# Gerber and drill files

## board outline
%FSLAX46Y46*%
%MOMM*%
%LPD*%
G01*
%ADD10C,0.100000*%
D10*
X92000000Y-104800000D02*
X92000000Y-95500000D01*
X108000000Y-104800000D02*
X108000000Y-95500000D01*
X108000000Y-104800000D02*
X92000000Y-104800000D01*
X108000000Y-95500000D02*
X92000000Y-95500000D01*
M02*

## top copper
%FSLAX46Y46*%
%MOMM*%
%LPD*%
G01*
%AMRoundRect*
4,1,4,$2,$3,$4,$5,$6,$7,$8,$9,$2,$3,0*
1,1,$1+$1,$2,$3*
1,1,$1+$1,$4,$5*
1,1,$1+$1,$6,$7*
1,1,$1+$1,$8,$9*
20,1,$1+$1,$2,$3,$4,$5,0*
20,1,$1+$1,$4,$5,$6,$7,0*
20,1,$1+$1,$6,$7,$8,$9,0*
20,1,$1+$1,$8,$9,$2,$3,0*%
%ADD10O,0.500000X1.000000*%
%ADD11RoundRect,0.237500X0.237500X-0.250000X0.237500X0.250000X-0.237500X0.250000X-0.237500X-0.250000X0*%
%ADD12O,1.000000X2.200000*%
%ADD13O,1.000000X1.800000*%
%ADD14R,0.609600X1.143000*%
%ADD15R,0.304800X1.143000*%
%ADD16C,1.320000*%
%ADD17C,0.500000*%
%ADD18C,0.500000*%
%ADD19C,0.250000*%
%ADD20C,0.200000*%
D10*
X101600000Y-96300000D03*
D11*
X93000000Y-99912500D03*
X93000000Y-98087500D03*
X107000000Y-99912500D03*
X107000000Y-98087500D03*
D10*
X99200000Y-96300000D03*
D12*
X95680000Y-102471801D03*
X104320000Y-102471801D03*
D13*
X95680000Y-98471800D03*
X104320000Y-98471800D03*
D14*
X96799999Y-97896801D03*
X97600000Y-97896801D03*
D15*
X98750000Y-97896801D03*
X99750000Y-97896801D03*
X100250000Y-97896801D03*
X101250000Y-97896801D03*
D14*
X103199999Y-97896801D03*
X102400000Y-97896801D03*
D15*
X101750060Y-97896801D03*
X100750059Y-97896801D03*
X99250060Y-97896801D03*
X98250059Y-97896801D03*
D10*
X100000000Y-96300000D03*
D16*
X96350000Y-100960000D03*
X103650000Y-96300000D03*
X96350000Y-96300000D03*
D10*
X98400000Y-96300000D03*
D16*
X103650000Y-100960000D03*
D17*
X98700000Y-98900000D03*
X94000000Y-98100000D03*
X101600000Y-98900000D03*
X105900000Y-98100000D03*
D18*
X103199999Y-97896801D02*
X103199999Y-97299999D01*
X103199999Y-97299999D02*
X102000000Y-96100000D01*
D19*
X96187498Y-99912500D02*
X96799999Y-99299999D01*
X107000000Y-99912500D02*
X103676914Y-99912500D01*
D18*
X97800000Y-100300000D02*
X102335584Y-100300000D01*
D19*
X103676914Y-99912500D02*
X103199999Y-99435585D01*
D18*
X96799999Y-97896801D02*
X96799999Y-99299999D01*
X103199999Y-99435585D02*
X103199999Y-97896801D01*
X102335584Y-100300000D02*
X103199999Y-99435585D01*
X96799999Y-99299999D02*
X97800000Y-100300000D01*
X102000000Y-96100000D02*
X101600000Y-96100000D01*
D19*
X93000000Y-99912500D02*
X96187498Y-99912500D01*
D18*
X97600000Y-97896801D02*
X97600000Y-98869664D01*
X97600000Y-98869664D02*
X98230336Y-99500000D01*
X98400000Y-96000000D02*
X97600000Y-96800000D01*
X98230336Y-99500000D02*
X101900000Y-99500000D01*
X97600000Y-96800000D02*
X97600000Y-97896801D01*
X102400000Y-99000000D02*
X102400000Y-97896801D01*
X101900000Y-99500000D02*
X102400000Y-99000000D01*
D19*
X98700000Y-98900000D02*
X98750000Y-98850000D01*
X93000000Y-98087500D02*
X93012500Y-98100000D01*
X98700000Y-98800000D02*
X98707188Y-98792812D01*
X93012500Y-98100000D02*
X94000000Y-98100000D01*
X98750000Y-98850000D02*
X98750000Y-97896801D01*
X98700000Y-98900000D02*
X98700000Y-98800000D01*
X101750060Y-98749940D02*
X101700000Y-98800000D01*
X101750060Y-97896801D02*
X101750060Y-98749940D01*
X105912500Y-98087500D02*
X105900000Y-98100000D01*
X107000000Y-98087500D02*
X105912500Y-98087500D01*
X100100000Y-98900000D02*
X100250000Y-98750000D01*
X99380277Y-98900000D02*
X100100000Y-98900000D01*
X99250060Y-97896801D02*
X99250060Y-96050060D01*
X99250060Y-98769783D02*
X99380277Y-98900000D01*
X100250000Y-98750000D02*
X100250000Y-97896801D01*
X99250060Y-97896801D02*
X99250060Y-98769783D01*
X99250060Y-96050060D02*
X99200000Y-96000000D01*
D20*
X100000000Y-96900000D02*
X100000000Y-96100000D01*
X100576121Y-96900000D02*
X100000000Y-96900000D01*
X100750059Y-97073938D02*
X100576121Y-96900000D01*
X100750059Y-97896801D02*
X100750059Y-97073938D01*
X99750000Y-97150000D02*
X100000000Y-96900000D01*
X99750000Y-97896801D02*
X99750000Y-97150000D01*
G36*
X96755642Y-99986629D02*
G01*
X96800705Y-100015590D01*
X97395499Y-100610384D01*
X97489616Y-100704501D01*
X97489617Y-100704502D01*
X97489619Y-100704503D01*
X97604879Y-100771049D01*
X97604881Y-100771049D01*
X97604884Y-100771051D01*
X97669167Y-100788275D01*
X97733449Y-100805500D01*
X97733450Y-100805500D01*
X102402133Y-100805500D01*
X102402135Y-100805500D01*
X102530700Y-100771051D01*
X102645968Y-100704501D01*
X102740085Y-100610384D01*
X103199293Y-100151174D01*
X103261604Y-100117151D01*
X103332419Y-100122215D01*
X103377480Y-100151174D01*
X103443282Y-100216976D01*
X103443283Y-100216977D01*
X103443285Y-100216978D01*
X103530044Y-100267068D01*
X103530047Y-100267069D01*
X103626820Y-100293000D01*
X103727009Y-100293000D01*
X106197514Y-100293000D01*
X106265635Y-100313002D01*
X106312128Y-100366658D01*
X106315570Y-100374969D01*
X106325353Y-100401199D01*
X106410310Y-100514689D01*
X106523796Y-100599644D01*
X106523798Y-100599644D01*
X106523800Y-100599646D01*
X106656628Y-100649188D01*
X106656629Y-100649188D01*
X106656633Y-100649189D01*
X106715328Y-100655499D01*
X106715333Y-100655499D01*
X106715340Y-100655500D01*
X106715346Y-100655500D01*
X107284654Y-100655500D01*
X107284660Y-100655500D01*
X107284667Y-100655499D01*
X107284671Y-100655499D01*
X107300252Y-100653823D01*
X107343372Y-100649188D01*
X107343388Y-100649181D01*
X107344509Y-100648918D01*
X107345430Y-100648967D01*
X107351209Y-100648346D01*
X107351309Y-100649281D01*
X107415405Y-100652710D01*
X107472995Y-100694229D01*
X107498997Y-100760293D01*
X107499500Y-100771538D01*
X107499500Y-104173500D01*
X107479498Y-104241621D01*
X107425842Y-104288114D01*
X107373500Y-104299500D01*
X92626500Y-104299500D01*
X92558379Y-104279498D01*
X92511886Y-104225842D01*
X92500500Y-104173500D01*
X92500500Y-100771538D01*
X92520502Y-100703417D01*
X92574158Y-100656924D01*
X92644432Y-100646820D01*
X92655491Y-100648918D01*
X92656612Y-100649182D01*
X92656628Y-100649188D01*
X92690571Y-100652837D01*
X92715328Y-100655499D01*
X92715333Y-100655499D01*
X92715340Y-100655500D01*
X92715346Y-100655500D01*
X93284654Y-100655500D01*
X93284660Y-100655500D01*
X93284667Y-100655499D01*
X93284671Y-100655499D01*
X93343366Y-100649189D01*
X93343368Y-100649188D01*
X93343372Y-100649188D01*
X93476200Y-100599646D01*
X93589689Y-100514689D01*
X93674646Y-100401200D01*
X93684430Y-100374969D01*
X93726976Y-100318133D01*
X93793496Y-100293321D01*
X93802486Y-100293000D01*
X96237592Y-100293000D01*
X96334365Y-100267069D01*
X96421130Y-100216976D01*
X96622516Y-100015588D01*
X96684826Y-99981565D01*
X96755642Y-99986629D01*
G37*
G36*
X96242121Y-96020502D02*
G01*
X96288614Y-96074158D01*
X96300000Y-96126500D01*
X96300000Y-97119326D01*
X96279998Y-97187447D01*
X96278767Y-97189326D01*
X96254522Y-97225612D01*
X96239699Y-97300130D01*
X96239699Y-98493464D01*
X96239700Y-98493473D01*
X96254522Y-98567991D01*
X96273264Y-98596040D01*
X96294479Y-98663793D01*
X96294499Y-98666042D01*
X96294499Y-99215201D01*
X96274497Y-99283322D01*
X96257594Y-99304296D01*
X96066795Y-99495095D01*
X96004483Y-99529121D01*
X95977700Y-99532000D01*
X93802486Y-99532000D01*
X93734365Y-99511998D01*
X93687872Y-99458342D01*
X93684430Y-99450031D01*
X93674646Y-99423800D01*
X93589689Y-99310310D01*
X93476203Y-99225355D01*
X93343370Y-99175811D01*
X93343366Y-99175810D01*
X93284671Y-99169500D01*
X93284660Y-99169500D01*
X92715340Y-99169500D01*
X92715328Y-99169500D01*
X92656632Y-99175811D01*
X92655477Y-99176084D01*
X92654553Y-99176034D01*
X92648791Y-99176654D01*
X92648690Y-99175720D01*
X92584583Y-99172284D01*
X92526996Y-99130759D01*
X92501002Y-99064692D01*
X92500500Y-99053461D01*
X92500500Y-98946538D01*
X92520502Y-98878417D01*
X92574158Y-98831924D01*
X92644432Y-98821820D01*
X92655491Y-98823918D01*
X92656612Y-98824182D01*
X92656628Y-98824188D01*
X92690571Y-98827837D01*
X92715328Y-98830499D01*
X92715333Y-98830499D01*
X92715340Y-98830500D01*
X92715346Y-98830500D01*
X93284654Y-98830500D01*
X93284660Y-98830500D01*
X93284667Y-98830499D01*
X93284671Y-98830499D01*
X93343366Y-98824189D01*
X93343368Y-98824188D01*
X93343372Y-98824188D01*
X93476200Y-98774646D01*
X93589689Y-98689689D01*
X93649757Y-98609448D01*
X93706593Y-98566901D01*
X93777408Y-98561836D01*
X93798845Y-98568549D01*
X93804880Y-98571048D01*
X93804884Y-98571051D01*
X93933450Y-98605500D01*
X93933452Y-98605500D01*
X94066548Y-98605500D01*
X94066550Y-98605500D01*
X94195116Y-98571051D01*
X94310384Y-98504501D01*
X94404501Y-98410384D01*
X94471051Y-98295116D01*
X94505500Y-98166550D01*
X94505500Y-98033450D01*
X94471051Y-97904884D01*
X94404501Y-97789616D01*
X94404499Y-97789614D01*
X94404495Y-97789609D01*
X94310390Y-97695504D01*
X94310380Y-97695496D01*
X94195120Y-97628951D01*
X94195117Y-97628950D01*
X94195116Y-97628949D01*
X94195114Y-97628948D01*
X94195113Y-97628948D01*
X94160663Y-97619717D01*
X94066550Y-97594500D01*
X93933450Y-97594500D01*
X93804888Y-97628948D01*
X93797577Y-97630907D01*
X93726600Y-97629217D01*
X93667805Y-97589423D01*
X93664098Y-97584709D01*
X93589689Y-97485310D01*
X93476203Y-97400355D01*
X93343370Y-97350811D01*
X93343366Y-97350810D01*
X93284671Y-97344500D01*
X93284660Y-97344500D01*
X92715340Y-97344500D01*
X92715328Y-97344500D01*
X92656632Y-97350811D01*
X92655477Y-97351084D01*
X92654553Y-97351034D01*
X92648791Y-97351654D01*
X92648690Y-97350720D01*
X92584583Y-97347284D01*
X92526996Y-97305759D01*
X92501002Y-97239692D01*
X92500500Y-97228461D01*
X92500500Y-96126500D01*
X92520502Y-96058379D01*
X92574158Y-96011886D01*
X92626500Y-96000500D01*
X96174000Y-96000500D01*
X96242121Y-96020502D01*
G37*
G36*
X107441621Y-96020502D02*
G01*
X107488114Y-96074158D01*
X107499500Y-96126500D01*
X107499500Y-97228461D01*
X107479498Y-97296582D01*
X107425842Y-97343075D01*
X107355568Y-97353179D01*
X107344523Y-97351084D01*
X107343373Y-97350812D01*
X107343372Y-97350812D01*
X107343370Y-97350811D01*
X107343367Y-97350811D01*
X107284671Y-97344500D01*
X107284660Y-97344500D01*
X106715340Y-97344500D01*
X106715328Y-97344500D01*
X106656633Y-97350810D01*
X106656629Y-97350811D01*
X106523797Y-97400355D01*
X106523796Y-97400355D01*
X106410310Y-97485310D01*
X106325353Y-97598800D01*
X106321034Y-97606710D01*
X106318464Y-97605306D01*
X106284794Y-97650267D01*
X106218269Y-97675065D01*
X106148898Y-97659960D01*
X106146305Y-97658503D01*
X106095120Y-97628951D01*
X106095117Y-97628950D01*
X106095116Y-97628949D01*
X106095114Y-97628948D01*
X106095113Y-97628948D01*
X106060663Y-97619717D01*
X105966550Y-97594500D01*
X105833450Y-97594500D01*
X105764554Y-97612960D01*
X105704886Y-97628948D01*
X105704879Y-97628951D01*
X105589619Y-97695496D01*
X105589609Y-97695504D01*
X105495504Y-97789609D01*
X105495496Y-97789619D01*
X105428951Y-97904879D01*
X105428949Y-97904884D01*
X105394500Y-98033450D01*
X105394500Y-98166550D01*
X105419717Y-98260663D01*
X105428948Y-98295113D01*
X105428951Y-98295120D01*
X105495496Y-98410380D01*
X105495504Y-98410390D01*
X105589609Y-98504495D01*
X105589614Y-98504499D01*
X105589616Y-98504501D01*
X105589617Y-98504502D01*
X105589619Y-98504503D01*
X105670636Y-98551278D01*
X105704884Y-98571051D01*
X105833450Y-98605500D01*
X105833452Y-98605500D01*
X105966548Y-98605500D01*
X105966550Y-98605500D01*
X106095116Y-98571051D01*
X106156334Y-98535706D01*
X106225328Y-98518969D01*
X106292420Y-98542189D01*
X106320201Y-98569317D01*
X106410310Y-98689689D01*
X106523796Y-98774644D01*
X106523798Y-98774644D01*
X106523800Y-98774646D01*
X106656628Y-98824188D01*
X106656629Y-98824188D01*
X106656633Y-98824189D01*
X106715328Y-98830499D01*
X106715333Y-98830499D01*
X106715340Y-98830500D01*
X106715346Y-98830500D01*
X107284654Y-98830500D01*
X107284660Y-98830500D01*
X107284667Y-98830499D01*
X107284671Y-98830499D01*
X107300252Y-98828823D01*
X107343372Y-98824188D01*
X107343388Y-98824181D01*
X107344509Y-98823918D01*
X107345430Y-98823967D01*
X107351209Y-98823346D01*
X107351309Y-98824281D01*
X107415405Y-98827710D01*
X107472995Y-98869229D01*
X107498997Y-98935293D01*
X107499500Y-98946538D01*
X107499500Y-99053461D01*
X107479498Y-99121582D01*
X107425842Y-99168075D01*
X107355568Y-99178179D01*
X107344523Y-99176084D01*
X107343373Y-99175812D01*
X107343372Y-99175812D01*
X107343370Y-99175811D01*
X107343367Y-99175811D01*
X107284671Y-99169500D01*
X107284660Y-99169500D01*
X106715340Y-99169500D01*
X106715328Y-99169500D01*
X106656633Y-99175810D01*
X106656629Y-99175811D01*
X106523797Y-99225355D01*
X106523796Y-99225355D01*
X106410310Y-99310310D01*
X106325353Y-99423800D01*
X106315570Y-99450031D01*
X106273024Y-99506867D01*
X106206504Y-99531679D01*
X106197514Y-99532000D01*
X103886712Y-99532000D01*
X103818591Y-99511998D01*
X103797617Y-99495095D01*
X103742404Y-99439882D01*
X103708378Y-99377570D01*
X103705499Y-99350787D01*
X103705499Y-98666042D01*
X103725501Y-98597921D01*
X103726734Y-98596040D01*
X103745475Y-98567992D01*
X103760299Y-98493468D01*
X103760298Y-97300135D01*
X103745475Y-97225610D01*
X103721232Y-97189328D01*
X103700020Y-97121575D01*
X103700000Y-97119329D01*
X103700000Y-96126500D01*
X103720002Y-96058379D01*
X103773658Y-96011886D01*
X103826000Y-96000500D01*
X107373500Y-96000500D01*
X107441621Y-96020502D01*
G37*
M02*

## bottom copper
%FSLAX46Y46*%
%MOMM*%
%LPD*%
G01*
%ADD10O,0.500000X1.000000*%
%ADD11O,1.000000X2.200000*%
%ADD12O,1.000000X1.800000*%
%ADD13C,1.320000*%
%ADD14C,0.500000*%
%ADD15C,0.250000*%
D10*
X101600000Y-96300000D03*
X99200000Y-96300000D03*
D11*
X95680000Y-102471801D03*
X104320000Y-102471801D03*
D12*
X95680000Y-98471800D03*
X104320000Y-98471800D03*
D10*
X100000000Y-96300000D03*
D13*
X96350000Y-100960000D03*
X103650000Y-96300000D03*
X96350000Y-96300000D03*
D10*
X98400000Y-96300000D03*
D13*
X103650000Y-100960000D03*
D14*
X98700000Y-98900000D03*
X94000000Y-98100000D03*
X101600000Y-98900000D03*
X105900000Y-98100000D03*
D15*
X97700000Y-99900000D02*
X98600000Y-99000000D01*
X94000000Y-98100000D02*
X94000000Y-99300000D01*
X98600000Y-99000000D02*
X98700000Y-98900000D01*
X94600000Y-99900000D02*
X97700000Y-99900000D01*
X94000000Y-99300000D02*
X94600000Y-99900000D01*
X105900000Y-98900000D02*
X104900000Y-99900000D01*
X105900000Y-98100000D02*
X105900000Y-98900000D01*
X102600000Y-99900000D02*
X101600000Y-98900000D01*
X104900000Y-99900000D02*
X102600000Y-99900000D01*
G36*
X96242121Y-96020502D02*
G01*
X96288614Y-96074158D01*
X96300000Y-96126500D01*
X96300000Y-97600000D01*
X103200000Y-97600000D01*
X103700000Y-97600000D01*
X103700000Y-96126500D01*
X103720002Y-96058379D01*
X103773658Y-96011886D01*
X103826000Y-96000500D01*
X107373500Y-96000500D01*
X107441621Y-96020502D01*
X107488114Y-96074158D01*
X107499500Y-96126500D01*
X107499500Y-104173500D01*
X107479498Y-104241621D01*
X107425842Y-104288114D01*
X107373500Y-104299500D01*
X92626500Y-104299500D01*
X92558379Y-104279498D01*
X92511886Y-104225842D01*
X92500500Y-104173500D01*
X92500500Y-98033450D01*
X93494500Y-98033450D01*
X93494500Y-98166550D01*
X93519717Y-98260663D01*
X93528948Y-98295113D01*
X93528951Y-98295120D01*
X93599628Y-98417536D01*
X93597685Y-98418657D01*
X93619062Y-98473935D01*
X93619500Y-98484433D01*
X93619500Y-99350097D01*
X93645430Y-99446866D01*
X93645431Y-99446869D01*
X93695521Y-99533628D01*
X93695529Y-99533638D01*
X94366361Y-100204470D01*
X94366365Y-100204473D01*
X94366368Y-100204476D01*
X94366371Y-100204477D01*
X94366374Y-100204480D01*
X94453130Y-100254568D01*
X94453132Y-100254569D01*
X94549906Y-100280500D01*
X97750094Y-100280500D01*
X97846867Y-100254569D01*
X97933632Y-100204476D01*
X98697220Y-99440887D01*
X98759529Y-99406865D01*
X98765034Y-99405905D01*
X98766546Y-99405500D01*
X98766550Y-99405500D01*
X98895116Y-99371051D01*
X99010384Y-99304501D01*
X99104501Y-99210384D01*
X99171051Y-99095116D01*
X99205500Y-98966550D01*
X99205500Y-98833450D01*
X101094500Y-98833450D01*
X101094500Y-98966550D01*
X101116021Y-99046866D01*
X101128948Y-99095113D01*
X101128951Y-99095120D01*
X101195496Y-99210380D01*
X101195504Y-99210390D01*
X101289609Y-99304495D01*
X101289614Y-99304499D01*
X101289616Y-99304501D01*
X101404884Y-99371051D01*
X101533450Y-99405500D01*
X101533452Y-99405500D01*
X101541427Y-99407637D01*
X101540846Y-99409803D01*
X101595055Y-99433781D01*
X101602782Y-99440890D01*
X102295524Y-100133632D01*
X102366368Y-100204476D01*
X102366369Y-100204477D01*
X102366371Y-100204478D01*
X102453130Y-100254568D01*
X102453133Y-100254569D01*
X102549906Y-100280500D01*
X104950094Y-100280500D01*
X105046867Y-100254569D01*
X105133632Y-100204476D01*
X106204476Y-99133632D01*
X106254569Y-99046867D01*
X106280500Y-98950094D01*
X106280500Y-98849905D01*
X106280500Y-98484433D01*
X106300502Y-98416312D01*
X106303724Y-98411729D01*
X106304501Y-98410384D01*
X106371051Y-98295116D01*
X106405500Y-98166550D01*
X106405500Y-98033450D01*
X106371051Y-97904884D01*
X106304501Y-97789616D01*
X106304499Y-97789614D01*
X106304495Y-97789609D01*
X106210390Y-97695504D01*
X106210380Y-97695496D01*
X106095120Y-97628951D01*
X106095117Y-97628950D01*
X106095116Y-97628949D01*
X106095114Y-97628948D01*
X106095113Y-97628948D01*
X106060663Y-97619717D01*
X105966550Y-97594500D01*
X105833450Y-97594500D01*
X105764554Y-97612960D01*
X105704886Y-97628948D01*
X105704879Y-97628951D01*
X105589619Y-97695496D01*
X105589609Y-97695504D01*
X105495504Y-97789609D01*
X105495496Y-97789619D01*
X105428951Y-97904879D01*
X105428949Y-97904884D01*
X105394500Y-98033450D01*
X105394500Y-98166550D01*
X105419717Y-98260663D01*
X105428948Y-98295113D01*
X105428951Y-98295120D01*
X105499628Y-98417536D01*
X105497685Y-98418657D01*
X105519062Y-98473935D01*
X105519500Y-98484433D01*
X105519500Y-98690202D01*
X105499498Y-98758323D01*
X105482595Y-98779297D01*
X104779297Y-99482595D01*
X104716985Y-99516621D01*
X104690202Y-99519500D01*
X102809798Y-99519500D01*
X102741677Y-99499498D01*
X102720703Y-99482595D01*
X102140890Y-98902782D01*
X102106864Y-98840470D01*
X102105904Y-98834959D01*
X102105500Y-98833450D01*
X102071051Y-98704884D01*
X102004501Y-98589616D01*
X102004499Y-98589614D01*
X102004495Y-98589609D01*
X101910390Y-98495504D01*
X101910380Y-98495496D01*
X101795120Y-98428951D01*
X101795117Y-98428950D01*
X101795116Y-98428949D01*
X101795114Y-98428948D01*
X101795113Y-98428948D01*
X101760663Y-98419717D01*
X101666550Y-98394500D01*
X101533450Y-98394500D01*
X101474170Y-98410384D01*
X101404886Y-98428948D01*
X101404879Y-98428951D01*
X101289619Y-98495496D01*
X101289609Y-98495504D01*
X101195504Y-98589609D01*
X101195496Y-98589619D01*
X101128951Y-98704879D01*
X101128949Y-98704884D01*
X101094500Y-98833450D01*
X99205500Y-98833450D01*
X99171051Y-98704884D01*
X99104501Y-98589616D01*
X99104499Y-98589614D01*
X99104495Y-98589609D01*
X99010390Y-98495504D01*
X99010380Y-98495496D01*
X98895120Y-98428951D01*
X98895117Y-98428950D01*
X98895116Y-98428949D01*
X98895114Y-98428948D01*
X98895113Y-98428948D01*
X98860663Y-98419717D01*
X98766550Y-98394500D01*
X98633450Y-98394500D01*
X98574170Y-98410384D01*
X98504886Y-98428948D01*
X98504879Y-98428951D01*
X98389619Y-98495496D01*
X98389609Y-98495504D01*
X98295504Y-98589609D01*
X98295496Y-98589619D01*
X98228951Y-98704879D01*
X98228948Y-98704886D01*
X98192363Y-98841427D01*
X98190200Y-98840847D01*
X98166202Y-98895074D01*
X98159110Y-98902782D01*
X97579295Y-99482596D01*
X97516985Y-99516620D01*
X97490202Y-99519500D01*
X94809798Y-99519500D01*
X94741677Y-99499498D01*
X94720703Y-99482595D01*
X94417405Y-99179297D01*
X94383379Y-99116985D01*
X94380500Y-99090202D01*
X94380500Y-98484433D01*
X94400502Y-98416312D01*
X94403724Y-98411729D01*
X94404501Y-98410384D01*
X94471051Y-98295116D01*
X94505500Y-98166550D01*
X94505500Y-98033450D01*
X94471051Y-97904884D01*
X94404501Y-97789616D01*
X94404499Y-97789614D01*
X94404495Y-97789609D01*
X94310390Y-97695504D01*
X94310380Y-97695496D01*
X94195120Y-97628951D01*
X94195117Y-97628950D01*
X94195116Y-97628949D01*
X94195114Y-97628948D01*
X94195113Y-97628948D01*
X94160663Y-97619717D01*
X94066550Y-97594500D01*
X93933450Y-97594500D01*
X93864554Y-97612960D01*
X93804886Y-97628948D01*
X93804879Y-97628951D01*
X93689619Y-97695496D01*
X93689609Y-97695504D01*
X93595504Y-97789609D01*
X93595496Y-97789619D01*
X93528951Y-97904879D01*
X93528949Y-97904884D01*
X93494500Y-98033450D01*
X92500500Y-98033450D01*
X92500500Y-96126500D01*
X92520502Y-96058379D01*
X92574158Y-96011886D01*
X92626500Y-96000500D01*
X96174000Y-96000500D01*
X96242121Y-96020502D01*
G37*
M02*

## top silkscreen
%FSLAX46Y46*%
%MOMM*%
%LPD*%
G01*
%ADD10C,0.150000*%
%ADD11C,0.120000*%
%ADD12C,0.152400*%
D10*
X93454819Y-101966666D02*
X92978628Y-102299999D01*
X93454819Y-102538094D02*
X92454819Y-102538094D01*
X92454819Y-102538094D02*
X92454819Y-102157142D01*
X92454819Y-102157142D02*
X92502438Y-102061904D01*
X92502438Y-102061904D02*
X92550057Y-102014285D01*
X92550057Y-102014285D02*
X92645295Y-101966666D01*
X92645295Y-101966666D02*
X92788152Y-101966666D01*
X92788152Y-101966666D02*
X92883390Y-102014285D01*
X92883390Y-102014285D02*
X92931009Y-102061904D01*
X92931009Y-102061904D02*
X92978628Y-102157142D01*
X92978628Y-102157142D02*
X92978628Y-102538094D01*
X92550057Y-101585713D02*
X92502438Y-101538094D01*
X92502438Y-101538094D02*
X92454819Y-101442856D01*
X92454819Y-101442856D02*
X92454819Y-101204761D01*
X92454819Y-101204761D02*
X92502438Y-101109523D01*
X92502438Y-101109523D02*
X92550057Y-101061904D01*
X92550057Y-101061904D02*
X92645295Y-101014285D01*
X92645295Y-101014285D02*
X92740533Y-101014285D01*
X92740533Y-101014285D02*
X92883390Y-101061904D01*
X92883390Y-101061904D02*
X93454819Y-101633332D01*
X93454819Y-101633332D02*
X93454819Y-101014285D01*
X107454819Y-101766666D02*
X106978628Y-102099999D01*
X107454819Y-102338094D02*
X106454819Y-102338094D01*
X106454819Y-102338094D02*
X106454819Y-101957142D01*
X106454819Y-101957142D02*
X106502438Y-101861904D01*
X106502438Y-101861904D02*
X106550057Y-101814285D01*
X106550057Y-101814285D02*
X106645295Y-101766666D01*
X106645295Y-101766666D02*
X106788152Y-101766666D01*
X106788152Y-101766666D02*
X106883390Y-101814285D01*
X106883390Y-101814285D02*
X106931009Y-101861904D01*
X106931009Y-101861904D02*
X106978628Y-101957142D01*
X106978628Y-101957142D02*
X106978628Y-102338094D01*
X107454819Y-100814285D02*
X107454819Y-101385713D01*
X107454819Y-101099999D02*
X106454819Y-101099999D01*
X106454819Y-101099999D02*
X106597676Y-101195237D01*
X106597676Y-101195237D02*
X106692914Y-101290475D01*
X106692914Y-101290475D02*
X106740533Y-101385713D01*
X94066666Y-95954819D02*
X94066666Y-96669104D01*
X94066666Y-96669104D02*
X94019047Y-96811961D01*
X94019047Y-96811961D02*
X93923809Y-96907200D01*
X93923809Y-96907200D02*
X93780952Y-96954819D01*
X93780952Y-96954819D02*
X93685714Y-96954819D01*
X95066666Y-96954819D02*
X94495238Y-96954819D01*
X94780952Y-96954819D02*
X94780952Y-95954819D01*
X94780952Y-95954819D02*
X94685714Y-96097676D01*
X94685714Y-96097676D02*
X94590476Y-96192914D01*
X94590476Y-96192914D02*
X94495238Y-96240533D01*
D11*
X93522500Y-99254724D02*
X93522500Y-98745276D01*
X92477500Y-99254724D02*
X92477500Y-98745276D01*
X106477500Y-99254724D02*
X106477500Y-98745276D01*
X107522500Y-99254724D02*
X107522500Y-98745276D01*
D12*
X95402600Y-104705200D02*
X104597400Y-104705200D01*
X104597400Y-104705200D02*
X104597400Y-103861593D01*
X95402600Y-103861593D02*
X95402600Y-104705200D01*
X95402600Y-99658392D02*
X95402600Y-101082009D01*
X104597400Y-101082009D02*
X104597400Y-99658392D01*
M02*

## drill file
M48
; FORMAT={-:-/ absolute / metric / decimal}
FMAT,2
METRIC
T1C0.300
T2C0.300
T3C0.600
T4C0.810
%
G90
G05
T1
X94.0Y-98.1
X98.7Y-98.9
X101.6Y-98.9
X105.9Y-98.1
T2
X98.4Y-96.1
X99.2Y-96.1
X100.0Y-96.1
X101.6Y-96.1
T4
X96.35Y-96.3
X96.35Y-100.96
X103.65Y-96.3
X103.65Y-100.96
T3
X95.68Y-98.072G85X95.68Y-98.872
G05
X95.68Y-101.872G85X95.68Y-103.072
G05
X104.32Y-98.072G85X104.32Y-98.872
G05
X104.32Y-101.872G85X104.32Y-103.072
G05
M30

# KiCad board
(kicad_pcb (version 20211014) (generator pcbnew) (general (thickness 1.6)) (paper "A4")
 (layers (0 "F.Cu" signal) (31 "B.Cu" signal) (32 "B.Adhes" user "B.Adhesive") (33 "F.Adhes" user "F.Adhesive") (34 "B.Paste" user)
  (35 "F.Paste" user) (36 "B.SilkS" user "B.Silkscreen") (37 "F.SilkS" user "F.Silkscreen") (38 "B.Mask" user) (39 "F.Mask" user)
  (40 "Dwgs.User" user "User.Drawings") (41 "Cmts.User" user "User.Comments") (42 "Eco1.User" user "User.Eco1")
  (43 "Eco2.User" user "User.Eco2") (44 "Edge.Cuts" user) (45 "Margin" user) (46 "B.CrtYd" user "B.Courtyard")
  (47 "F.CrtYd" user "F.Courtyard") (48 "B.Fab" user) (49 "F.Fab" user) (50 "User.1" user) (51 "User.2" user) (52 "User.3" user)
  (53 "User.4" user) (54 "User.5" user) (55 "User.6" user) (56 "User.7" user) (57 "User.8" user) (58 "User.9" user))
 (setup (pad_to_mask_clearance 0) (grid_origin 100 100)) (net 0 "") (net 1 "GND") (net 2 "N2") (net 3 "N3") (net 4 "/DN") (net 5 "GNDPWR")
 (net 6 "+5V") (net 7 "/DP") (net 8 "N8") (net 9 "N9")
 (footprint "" (layer "F.Cu") (at 101.6 96.1)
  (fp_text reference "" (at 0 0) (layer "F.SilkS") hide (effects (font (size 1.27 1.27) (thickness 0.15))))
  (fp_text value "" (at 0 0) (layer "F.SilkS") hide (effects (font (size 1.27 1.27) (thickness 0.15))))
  (pad "B11" thru_hole oval (at 0 0) (size 0.5 1) (drill 0.3 (offset 0 0.2)) (layers *.Cu *.Mask) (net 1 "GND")))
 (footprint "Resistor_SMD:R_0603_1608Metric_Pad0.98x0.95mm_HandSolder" (layer "F.Cu") (at 93 99 90)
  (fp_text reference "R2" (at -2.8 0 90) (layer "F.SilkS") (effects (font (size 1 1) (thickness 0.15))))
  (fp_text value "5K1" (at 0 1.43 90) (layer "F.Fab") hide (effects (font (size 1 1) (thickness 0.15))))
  (fp_line (start -0.254724 0.5225) (end 0.254724 0.5225) (layer "F.SilkS") (width 0.12))
  (fp_line (start -0.254724 -0.5225) (end 0.254724 -0.5225) (layer "F.SilkS") (width 0.12))
  (pad "1" smd roundrect (at -0.9125 0 90) (size 0.975 0.95) (layers "F.Cu" "F.Paste" "F.Mask") (roundrect_rratio 0.25) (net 1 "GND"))
  (pad "2" smd roundrect (at 0.9125 0 90) (size 0.975 0.95) (layers "F.Cu" "F.Paste" "F.Mask") (roundrect_rratio 0.25) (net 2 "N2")))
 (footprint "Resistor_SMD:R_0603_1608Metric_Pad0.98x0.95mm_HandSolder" (layer "F.Cu") (at 107 99 90)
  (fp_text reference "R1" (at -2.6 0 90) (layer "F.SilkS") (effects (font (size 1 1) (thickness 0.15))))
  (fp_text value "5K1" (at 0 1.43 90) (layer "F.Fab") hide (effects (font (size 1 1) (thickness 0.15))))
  (fp_line (start -0.254724 -0.5225) (end 0.254724 -0.5225) (layer "F.SilkS") (width 0.12))
  (fp_line (start -0.254724 0.5225) (end 0.254724 0.5225) (layer "F.SilkS") (width 0.12))
  (pad "1" smd roundrect (at -0.9125 0 90) (size 0.975 0.95) (layers "F.Cu" "F.Paste" "F.Mask") (roundrect_rratio 0.25) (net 1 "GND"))
  (pad "2" smd roundrect (at 0.9125 0 90) (size 0.975 0.95) (layers "F.Cu" "F.Paste" "F.Mask") (roundrect_rratio 0.25) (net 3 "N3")))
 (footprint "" (layer "F.Cu") (at 99.2 96.1)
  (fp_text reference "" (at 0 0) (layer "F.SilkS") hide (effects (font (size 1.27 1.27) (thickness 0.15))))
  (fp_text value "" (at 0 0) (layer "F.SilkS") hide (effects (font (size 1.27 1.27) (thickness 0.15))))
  (pad "B9" thru_hole oval (at 0 0) (size 0.5 1) (drill 0.3 (offset 0 0.2)) (layers *.Cu *.Mask) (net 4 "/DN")))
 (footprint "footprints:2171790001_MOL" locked (layer "F.Cu") (at 100 101.2)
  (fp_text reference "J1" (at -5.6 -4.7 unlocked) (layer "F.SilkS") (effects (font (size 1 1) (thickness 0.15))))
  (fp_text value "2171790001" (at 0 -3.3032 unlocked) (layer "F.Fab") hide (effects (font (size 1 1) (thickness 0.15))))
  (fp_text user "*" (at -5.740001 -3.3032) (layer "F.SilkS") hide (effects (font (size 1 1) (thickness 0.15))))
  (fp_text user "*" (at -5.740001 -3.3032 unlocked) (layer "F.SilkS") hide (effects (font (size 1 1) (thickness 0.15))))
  (fp_line (start -4.5974 3.5052) (end 4.5974 3.5052) (layer "F.SilkS") (width 0.1524))
  (fp_line (start 4.5974 3.5052) (end 4.5974 2.661593) (layer "F.SilkS") (width 0.1524))
  (fp_line (start -4.5974 2.661593) (end -4.5974 3.5052) (layer "F.SilkS") (width 0.1524))
  (fp_line (start -4.5974 -1.541608) (end -4.5974 -0.117991) (layer "F.SilkS") (width 0.1524))
  (fp_line (start 4.5974 -0.117991) (end 4.5974 -1.541608) (layer "F.SilkS") (width 0.1524))
  (pad "13" thru_hole oval locked (at -4.32 1.271801) (size 1 2.2) (drill oval 0.6 1.8) (layers *.Cu *.Mask) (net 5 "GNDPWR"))
  (pad "14" thru_hole oval locked (at 4.32 1.271801) (size 1 2.2) (drill oval 0.6 1.8) (layers *.Cu *.Mask) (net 5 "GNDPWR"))
  (pad "15" thru_hole oval locked (at -4.32 -2.7282) (size 1 1.8) (drill oval 0.6 1.4) (layers *.Cu *.Mask) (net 5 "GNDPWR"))
  (pad "16" thru_hole oval locked (at 4.32 -2.7282) (size 1 1.8) (drill oval 0.6 1.4) (layers *.Cu *.Mask) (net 5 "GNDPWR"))
  (pad "A1/B12" smd rect locked (at -3.200001 -3.303199) (size 0.6096 1.143) (layers "F.Cu" "F.Paste" "F.Mask") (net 1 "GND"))
  (pad "A4/B9" smd rect locked (at -2.4 -3.303199) (size 0.6096 1.143) (layers "F.Cu" "F.Paste" "F.Mask") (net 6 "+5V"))
  (pad "A5" smd rect locked (at -1.25 -3.303199) (size 0.3048 1.143) (layers "F.Cu" "F.Paste" "F.Mask") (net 2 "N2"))
  (pad "A6" smd rect locked (at -0.25 -3.303199) (size 0.3048 1.143) (layers "F.Cu" "F.Paste" "F.Mask") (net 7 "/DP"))
  (pad "A7" smd rect locked (at 0.25 -3.303199) (size 0.3048 1.143) (layers "F.Cu" "F.Paste" "F.Mask") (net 4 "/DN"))
  (pad "A8" smd rect locked (at 1.25 -3.303199) (size 0.3048 1.143) (layers "F.Cu" "F.Paste" "F.Mask") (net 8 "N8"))
  (pad "B1/A12" smd rect locked (at 3.199999 -3.303199) (size 0.6096 1.143) (layers "F.Cu" "F.Paste" "F.Mask") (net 1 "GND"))
  (pad "B4/A9" smd rect locked (at 2.4 -3.303199) (size 0.6096 1.143) (layers "F.Cu" "F.Paste" "F.Mask") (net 6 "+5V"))
  (pad "B5" smd rect locked (at 1.75006 -3.303199) (size 0.3048 1.143) (layers "F.Cu" "F.Paste" "F.Mask") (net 3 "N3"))
  (pad "B6" smd rect locked (at 0.750059 -3.303199) (size 0.3048 1.143) (layers "F.Cu" "F.Paste" "F.Mask") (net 7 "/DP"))
  (pad "B7" smd rect locked (at -0.74994 -3.303199) (size 0.3048 1.143) (layers "F.Cu" "F.Paste" "F.Mask") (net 4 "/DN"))
  (pad "B8" smd rect locked (at -1.749941 -3.303199) (size 0.3048 1.143) (layers "F.Cu" "F.Paste" "F.Mask") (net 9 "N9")))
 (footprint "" (layer "F.Cu") (at 100 96.1)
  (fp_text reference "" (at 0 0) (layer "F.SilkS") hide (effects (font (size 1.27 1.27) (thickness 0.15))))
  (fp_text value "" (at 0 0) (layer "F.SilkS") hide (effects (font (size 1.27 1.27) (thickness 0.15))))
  (pad "B10" thru_hole oval (at 0 0) (size 0.5 1) (drill 0.3 (offset 0 0.2)) (layers *.Cu *.Mask) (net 7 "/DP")))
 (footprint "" (layer "F.Cu") (at 96.35 100.96)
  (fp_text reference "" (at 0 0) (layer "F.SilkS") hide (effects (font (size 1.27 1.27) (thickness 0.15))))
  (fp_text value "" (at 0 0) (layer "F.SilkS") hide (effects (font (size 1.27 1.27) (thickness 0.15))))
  (pad "B12" thru_hole circle (at 0 0) (size 1.32 1.32) (drill 0.81) (layers *.Cu *.Mask) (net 5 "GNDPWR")))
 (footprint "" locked (layer "F.Cu") (at 103.65 96.3)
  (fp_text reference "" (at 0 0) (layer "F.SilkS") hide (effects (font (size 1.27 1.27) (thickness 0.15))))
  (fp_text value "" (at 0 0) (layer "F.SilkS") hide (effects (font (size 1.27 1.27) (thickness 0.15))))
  (pad "B12" thru_hole circle locked (at 0 0) (size 1.32 1.32) (drill 0.81) (layers *.Cu *.Mask) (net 5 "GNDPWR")))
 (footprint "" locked (layer "F.Cu") (at 96.35 96.3)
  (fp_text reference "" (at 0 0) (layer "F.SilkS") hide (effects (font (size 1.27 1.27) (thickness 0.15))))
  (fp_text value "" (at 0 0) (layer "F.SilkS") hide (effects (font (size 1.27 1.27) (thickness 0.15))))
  (pad "B12" thru_hole circle locked (at 0 0) (size 1.32 1.32) (drill 0.81) (layers *.Cu *.Mask) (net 5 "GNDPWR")))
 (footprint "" (layer "F.Cu") (at 98.4 96.1)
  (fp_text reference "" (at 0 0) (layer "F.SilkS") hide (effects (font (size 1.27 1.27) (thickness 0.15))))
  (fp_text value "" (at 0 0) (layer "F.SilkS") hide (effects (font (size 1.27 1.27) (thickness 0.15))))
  (pad "B8" thru_hole oval (at 0 0) (size 0.5 1) (drill 0.3 (offset 0 0.2)) (layers *.Cu *.Mask) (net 6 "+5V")))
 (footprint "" (layer "F.Cu") (at 103.65 100.96)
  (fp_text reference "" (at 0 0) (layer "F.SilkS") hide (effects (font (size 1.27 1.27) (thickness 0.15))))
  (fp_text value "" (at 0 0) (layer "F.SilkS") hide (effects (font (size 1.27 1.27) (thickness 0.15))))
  (pad "B12" thru_hole circle (at 0 0) (size 1.32 1.32) (drill 0.81) (layers *.Cu *.Mask) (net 5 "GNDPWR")))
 (gr_line (start 92 104.8) (end 92 95.5) (layer "Edge.Cuts") (width 0.1))
 (gr_line (start 108 104.8) (end 108 95.5) (layer "Edge.Cuts") (width 0.1))
 (gr_line (start 108 104.8) (end 92 104.8) (layer "Edge.Cuts") (width 0.1))
 (gr_line (start 108 95.5) (end 92 95.5) (layer "Edge.Cuts") (width 0.1))
 (segment (start 103.199999 97.896801) (end 103.199999 97.299999) (width 0.5) (layer "F.Cu") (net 1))
 (segment (start 103.199999 97.299999) (end 102 96.1) (width 0.5) (layer "F.Cu") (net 1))
 (segment (start 96.187498 99.9125) (end 96.799999 99.299999) (width 0.25) (layer "F.Cu") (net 1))
 (segment (start 107 99.9125) (end 103.676914 99.9125) (width 0.25) (layer "F.Cu") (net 1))
 (segment (start 97.8 100.3) (end 102.335584 100.3) (width 0.5) (layer "F.Cu") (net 1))
 (segment (start 103.676914 99.9125) (end 103.199999 99.435585) (width 0.25) (layer "F.Cu") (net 1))
 (segment (start 96.799999 97.896801) (end 96.799999 99.299999) (width 0.5) (layer "F.Cu") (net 1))
 (segment (start 103.199999 99.435585) (end 103.199999 97.896801) (width 0.5) (layer "F.Cu") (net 1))
 (segment (start 102.335584 100.3) (end 103.199999 99.435585) (width 0.5) (layer "F.Cu") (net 1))
 (segment (start 96.799999 99.299999) (end 97.8 100.3) (width 0.5) (layer "F.Cu") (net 1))
 (segment (start 102 96.1) (end 101.6 96.1) (width 0.5) (layer "F.Cu") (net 1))
 (segment (start 93 99.9125) (end 96.187498 99.9125) (width 0.25) (layer "F.Cu") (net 1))
 (segment (start 97.6 97.896801) (end 97.6 98.869664) (width 0.5) (layer "F.Cu") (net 6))
 (segment (start 97.6 98.869664) (end 98.230336 99.5) (width 0.5) (layer "F.Cu") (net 6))
 (segment (start 98.4 96) (end 97.6 96.8) (width 0.5) (layer "F.Cu") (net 6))
 (segment (start 98.230336 99.5) (end 101.9 99.5) (width 0.5) (layer "F.Cu") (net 6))
 (segment (start 97.6 96.8) (end 97.6 97.896801) (width 0.5) (layer "F.Cu") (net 6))
 (segment (start 102.4 99) (end 102.4 97.896801) (width 0.5) (layer "F.Cu") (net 6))
 (segment (start 101.9 99.5) (end 102.4 99) (width 0.5) (layer "F.Cu") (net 6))
 (segment (start 98.7 98.9) (end 98.75 98.85) (width 0.25) (layer "F.Cu") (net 2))
 (segment (start 93 98.0875) (end 93.0125 98.1) (width 0.25) (layer "F.Cu") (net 2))
 (segment (start 98.7 98.8) (end 98.707188 98.792812) (width 0.25) (layer "F.Cu") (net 2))
 (segment (start 93.0125 98.1) (end 94 98.1) (width 0.25) (layer "F.Cu") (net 2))
 (segment (start 98.75 98.85) (end 98.75 97.896801) (width 0.25) (layer "F.Cu") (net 2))
 (segment (start 98.7 98.9) (end 98.7 98.8) (width 0.25) (layer "F.Cu") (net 2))
 (via (at 98.7 98.9) (size 0.5) (drill 0.3) (layers "F.Cu" "B.Cu") (free) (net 2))
 (via (at 94 98.1) (size 0.5) (drill 0.3) (layers "F.Cu" "B.Cu") (free) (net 2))
 (segment (start 97.7 99.9) (end 98.6 99) (width 0.25) (layer "B.Cu") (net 2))
 (segment (start 94 98.1) (end 94 99.3) (width 0.25) (layer "B.Cu") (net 2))
 (segment (start 98.6 99) (end 98.7 98.9) (width 0.25) (layer "B.Cu") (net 2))
 (segment (start 94.6 99.9) (end 97.7 99.9) (width 0.25) (layer "B.Cu") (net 2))
 (segment (start 94 99.3) (end 94.6 99.9) (width 0.25) (layer "B.Cu") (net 2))
 (segment (start 101.75006 98.74994) (end 101.7 98.8) (width 0.25) (layer "F.Cu") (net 3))
 (segment (start 101.75006 97.896801) (end 101.75006 98.74994) (width 0.25) (layer "F.Cu") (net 3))
 (segment (start 105.9125 98.0875) (end 105.9 98.1) (width 0.25) (layer "F.Cu") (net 3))
 (segment (start 107 98.0875) (end 105.9125 98.0875) (width 0.25) (layer "F.Cu") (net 3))
 (via (at 101.6 98.9) (size 0.5) (drill 0.3) (layers "F.Cu" "B.Cu") (free) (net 3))
 (via (at 105.9 98.1) (size 0.5) (drill 0.3) (layers "F.Cu" "B.Cu") (free) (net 3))
 (segment (start 105.9 98.9) (end 104.9 99.9) (width 0.25) (layer "B.Cu") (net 3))
 (segment (start 105.9 98.1) (end 105.9 98.9) (width 0.25) (layer "B.Cu") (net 3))
 (segment (start 102.6 99.9) (end 101.6 98.9) (width 0.25) (layer "B.Cu") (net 3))
 (segment (start 104.9 99.9) (end 102.6 99.9) (width 0.25) (layer "B.Cu") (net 3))
 (segment (start 100.1 98.9) (end 100.25 98.75) (width 0.25) (layer "F.Cu") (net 4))
 (segment (start 99.380277 98.9) (end 100.1 98.9) (width 0.25) (layer "F.Cu") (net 4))
 (segment (start 99.25006 97.896801) (end 99.25006 96.05006) (width 0.25) (layer "F.Cu") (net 4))
 (segment (start 99.25006 98.769783) (end 99.380277 98.9) (width 0.25) (layer "F.Cu") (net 4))
 (segment (start 100.25 98.75) (end 100.25 97.896801) (width 0.25) (layer "F.Cu") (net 4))
 (segment (start 99.25006 97.896801) (end 99.25006 98.769783) (width 0.25) (layer "F.Cu") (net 4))
 (segment (start 99.25006 96.05006) (end 99.2 96) (width 0.25) (layer "F.Cu") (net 4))
 (segment (start 100 96.9) (end 100 96.1) (width 0.2) (layer "F.Cu") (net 7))
 (segment (start 100.576121 96.9) (end 100 96.9) (width 0.2) (layer "F.Cu") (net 7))
 (segment (start 100.750059 97.073938) (end 100.576121 96.9) (width 0.2) (layer "F.Cu") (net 7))
 (segment (start 100.750059 97.896801) (end 100.750059 97.073938) (width 0.2) (layer "F.Cu") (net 7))
 (segment (start 99.75 97.15) (end 100 96.9) (width 0.2) (layer "F.Cu") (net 7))
 (segment (start 99.75 97.896801) (end 99.75 97.15) (width 0.2) (layer "F.Cu") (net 7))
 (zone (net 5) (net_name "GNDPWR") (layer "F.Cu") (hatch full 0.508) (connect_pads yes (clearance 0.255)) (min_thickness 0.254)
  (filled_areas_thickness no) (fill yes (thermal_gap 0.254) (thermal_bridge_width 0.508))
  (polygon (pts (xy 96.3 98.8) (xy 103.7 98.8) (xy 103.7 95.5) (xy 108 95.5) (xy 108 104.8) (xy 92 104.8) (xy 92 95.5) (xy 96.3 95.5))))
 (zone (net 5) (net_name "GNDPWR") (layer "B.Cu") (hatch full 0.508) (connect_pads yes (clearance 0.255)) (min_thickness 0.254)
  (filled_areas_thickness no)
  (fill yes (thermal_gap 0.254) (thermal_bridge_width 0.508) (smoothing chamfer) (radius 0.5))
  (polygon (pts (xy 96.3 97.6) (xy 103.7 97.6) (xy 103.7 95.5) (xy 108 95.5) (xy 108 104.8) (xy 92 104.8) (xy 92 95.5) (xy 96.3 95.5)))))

